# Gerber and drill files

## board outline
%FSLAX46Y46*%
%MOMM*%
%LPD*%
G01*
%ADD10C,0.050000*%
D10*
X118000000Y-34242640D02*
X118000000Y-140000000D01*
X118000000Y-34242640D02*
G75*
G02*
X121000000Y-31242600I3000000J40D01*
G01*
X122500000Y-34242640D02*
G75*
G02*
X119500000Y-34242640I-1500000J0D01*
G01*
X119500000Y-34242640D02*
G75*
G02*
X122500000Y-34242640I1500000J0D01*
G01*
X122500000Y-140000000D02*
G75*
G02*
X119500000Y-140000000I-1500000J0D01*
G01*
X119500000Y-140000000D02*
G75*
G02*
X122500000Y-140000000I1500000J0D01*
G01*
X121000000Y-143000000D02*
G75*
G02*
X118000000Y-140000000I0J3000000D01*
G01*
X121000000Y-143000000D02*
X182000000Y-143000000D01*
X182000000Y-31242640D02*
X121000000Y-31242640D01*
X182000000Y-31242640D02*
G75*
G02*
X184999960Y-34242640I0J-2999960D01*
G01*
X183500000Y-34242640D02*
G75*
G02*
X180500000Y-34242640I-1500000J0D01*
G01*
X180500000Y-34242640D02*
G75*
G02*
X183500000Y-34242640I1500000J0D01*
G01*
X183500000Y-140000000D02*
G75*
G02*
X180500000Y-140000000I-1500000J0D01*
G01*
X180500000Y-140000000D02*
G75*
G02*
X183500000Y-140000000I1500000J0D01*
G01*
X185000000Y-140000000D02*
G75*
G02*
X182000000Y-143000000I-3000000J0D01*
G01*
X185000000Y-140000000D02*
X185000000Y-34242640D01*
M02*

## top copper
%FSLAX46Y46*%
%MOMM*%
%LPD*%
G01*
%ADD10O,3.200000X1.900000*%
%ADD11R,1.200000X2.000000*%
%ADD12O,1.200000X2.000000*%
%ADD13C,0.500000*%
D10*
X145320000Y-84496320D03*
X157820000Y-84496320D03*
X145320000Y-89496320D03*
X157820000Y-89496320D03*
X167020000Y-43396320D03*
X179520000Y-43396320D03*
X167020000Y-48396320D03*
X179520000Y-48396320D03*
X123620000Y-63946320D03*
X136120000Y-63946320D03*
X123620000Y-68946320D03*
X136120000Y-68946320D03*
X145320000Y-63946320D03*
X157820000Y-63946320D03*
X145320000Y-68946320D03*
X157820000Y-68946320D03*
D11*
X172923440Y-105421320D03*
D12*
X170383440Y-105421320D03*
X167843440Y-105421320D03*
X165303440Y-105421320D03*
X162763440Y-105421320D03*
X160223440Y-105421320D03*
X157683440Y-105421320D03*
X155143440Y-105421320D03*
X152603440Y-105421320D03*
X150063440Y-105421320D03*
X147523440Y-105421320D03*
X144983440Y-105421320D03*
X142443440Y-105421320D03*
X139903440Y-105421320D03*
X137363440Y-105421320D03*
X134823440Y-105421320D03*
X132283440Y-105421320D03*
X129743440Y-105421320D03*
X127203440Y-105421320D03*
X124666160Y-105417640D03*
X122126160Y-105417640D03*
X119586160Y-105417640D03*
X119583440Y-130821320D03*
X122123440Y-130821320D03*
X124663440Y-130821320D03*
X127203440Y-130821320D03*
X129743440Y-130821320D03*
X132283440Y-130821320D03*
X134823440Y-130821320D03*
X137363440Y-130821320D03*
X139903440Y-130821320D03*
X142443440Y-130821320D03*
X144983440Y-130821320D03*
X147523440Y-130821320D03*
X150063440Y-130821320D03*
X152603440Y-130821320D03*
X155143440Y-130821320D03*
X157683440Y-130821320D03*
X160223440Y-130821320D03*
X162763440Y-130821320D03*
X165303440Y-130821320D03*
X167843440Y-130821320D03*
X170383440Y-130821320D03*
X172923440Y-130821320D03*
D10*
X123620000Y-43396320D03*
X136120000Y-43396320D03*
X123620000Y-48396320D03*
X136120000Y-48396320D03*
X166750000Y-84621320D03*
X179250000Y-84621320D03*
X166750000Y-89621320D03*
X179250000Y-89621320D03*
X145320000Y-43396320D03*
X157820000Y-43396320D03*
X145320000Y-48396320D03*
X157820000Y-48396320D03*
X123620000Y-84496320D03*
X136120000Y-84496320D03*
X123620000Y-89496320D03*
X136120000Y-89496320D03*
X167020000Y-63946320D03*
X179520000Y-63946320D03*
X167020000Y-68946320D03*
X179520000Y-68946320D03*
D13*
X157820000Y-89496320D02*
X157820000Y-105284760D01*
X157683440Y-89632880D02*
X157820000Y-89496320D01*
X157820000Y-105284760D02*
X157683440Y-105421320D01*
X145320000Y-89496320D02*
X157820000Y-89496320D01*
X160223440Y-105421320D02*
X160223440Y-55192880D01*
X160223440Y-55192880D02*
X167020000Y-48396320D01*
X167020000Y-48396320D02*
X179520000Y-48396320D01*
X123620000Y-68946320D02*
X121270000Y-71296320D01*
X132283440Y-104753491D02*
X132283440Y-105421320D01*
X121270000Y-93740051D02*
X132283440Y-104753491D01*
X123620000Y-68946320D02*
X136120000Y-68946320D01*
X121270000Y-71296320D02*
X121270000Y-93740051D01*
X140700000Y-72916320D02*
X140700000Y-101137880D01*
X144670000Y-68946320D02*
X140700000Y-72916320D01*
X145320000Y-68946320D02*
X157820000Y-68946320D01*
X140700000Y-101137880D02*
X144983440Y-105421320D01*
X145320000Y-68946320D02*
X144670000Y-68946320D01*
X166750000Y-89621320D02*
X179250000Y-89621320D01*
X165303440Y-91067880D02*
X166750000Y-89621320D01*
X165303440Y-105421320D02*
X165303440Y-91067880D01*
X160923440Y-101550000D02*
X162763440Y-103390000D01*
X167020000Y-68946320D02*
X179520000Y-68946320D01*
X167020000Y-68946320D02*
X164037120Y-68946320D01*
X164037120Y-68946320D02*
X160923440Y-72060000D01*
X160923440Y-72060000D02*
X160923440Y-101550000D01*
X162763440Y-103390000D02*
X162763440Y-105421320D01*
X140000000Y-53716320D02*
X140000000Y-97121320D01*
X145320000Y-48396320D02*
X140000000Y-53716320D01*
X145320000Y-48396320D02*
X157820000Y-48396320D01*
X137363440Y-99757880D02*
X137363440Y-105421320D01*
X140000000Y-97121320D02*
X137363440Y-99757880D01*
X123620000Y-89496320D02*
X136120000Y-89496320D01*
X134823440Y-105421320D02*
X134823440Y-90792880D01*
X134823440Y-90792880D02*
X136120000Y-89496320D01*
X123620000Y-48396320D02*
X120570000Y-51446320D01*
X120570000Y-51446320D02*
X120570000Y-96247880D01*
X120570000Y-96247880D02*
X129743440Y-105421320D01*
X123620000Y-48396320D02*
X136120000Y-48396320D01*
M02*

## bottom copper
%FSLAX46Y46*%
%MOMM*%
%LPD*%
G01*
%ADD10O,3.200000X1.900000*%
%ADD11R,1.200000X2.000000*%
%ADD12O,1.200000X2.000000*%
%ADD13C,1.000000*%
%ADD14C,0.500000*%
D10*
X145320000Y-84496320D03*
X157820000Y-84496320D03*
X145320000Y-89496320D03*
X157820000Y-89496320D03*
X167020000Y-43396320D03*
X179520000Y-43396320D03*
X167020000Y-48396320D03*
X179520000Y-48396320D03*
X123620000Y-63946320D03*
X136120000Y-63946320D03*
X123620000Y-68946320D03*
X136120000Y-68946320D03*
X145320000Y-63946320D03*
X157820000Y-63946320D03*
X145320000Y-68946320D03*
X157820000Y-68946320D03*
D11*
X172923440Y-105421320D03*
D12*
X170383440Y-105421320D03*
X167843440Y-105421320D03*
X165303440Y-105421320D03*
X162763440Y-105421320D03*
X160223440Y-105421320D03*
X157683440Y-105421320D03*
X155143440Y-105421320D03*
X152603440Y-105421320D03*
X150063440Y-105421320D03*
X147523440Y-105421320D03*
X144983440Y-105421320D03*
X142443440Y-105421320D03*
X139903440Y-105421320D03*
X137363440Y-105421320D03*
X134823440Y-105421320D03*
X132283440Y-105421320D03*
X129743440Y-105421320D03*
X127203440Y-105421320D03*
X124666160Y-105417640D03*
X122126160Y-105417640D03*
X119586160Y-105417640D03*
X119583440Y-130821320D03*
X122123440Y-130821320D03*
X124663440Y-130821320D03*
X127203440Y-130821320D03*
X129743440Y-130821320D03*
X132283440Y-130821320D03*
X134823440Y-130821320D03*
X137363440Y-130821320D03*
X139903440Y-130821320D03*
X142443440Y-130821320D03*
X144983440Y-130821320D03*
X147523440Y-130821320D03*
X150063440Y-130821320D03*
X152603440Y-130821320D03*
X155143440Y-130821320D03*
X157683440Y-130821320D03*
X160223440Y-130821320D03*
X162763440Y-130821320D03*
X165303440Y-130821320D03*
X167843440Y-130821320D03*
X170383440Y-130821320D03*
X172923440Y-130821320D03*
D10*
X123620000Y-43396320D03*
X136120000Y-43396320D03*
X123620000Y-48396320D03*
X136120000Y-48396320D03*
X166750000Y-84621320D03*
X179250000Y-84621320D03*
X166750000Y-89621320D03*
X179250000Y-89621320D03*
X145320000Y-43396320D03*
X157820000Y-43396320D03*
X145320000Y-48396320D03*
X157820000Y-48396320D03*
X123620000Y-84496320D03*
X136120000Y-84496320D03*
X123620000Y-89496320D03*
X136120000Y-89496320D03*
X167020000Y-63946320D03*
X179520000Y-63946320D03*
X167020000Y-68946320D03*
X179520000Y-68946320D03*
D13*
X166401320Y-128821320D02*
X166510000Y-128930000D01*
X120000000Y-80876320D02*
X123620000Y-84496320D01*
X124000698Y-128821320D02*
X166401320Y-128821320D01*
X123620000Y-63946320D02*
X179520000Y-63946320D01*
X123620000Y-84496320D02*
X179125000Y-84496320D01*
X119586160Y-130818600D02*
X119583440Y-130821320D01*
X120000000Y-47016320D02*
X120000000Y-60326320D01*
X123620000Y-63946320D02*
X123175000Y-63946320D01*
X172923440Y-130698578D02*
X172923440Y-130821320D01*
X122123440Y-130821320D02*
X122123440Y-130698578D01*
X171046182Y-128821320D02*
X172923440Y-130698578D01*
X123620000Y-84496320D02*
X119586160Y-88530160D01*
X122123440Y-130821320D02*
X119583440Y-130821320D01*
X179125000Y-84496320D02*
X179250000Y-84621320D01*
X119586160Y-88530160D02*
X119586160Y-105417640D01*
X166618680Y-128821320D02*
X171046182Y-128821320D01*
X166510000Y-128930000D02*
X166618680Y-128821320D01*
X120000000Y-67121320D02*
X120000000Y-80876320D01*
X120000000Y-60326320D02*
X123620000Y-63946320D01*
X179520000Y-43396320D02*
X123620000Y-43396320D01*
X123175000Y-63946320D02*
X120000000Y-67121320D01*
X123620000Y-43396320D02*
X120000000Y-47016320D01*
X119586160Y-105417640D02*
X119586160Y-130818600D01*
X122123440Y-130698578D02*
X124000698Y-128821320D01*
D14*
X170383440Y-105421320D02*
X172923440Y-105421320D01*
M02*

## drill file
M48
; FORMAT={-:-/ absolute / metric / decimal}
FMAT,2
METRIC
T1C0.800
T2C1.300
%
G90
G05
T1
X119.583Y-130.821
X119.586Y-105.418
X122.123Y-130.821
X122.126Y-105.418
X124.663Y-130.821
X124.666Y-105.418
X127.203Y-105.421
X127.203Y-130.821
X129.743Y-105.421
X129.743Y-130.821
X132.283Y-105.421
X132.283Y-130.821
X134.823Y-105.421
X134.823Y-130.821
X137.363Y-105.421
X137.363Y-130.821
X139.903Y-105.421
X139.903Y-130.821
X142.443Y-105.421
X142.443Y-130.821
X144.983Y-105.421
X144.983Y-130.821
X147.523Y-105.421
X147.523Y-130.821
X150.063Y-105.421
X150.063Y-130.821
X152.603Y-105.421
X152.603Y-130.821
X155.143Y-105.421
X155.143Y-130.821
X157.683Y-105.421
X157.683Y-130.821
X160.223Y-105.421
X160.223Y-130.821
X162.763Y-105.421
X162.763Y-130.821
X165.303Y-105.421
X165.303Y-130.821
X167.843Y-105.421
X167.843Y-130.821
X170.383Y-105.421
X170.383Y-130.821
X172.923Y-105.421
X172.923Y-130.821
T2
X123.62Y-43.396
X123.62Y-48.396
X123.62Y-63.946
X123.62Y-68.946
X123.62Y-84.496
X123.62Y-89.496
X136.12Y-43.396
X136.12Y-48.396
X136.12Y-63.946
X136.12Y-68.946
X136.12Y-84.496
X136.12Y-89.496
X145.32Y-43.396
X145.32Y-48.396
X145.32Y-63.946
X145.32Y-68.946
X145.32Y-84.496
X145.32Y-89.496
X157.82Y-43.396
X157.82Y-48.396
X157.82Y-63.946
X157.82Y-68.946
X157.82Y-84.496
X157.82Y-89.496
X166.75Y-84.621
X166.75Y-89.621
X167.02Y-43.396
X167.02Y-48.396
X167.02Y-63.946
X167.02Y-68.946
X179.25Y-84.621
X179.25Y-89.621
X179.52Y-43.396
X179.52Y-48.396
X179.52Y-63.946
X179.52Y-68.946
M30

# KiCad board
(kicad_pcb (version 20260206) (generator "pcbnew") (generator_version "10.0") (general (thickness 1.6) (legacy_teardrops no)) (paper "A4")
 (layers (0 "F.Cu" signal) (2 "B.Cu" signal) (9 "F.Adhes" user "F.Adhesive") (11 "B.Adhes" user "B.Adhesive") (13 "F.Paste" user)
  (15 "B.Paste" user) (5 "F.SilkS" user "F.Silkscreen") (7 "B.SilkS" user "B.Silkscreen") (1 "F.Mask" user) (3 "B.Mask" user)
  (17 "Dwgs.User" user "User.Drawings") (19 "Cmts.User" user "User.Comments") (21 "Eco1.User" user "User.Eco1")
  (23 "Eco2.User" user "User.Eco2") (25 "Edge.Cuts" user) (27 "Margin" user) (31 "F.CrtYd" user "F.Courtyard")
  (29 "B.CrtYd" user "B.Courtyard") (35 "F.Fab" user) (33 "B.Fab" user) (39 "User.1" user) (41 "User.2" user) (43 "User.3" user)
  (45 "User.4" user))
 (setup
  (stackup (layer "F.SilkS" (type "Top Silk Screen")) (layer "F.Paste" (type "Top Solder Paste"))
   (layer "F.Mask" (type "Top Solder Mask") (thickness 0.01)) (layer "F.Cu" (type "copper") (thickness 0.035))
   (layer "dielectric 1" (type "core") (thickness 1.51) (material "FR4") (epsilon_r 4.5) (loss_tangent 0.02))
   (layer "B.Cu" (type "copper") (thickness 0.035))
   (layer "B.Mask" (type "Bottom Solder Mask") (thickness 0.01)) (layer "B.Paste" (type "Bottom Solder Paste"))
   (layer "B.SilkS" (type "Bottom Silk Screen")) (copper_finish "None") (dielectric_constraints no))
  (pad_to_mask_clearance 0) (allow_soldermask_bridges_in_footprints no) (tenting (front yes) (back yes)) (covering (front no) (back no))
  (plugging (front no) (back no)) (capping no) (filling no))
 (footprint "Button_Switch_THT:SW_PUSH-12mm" (layer "F.Cu") (at 145.32 84.49632)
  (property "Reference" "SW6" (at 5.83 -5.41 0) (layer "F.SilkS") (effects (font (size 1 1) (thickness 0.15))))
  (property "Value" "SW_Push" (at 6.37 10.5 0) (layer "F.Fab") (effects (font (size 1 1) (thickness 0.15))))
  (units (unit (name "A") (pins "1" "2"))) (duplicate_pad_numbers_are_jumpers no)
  (pad "1" thru_hole oval (at 0 0) (size 3.2 1.9) (drill 1.3) (layers "*.Cu" "*.Mask") (remove_unused_layers no) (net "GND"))
  (pad "1" thru_hole oval (at 12.5 0) (size 3.2 1.9) (drill 1.3) (layers "*.Cu" "*.Mask") (remove_unused_layers no) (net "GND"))
  (pad "2" thru_hole oval (at 0 5) (size 3.2 1.9) (drill 1.3) (layers "*.Cu" "*.Mask") (remove_unused_layers no)
   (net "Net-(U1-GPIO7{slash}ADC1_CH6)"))
  (pad "2" thru_hole oval (at 12.5 5) (size 3.2 1.9) (drill 1.3) (layers "*.Cu" "*.Mask") (remove_unused_layers no)
   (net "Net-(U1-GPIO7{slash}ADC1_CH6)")))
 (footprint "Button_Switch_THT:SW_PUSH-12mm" (layer "F.Cu") (at 167.02 43.39632)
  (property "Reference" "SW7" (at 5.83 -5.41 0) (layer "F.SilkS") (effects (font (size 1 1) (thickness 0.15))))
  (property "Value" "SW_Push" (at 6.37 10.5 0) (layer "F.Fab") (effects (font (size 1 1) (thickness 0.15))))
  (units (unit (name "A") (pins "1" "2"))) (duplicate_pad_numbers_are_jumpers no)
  (pad "1" thru_hole oval (at 0 0) (size 3.2 1.9) (drill 1.3) (layers "*.Cu" "*.Mask") (remove_unused_layers no) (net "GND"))
  (pad "1" thru_hole oval (at 12.5 0) (size 3.2 1.9) (drill 1.3) (layers "*.Cu" "*.Mask") (remove_unused_layers no) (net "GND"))
  (pad "2" thru_hole oval (at 0 5) (size 3.2 1.9) (drill 1.3) (layers "*.Cu" "*.Mask") (remove_unused_layers no)
   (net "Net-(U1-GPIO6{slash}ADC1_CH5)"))
  (pad "2" thru_hole oval (at 12.5 5) (size 3.2 1.9) (drill 1.3) (layers "*.Cu" "*.Mask") (remove_unused_layers no)
   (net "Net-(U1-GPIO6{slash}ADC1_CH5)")))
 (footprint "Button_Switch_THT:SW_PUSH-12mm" (layer "F.Cu") (at 123.62 63.94632)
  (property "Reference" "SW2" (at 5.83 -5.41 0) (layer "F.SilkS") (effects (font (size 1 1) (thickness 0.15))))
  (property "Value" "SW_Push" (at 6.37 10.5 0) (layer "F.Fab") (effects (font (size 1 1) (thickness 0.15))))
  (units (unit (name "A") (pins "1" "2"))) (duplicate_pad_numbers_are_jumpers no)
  (pad "1" thru_hole oval (at 0 0) (size 3.2 1.9) (drill 1.3) (layers "*.Cu" "*.Mask") (remove_unused_layers no) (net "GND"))
  (pad "1" thru_hole oval (at 12.5 0) (size 3.2 1.9) (drill 1.3) (layers "*.Cu" "*.Mask") (remove_unused_layers no) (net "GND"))
  (pad "2" thru_hole oval (at 0 5) (size 3.2 1.9) (drill 1.3) (layers "*.Cu" "*.Mask") (remove_unused_layers no)
   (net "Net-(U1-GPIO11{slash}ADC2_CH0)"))
  (pad "2" thru_hole oval (at 12.5 5) (size 3.2 1.9) (drill 1.3) (layers "*.Cu" "*.Mask") (remove_unused_layers no)
   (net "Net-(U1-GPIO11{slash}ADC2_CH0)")))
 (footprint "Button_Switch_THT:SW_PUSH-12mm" (layer "F.Cu") (at 145.32 63.94632)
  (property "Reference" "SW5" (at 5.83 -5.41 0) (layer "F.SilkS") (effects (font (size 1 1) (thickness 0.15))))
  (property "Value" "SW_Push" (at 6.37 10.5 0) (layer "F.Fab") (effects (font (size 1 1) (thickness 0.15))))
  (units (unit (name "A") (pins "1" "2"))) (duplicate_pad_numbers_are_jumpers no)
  (pad "1" thru_hole oval (at 0 0) (size 3.2 1.9) (drill 1.3) (layers "*.Cu" "*.Mask") (remove_unused_layers no) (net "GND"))
  (pad "1" thru_hole oval (at 12.5 0) (size 3.2 1.9) (drill 1.3) (layers "*.Cu" "*.Mask") (remove_unused_layers no) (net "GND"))
  (pad "2" thru_hole oval (at 0 5) (size 3.2 1.9) (drill 1.3) (layers "*.Cu" "*.Mask") (remove_unused_layers no)
   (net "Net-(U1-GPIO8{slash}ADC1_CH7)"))
  (pad "2" thru_hole oval (at 12.5 5) (size 3.2 1.9) (drill 1.3) (layers "*.Cu" "*.Mask") (remove_unused_layers no)
   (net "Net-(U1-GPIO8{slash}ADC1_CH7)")))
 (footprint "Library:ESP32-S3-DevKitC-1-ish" (layer "F.Cu") (at 172.92344 105.42132 -90)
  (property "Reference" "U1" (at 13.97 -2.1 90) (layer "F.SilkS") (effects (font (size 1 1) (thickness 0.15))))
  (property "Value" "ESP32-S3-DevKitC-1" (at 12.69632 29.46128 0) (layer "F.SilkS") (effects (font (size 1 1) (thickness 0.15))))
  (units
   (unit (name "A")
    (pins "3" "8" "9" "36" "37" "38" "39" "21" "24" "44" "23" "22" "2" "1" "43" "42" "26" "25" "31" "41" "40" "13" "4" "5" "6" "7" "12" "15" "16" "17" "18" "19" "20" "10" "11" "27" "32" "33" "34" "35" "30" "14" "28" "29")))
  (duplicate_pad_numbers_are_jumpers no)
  (pad "1" thru_hole rect (at 0 0 180) (size 1.2 2) (drill 0.8) (layers "*.Cu" "*.Mask") (remove_unused_layers no) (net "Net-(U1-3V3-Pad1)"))
  (pad "2" thru_hole oval (at 0 2.54 180) (size 1.2 2) (drill 0.8) (layers "*.Cu" "*.Mask") (remove_unused_layers no)
   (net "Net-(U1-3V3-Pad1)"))
  (pad "3" thru_hole oval (at 0 5.08 180) (size 1.2 2) (drill 0.8) (layers "*.Cu" "*.Mask") (remove_unused_layers no)
   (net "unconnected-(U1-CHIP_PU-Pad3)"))
  (pad "4" thru_hole oval (at 0 7.62 180) (size 1.2 2) (drill 0.8) (layers "*.Cu" "*.Mask") (remove_unused_layers no)
   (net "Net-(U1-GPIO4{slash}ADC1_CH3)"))
  (pad "5" thru_hole oval (at 0 10.16 180) (size 1.2 2) (drill 0.8) (layers "*.Cu" "*.Mask") (remove_unused_layers no)
   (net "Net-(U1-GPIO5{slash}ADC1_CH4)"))
  (pad "6" thru_hole oval (at 0 12.7 180) (size 1.2 2) (drill 0.8) (layers "*.Cu" "*.Mask") (remove_unused_layers no)
   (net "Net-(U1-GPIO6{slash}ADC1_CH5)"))
  (pad "7" thru_hole oval (at 0 15.24 180) (size 1.2 2) (drill 0.8) (layers "*.Cu" "*.Mask") (remove_unused_layers no)
   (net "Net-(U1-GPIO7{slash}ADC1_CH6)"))
  (pad "8" thru_hole oval (at 0 17.78 180) (size 1.2 2) (drill 0.8) (layers "*.Cu" "*.Mask") (remove_unused_layers no)
   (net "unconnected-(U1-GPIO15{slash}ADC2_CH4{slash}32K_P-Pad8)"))
  (pad "9" thru_hole oval (at 0 20.32 180) (size 1.2 2) (drill 0.8) (layers "*.Cu" "*.Mask") (remove_unused_layers no)
   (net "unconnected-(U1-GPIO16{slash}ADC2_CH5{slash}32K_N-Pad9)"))
  (pad "10" thru_hole oval (at 0 22.86 180) (size 1.2 2) (drill 0.8) (layers "*.Cu" "*.Mask") (remove_unused_layers no)
   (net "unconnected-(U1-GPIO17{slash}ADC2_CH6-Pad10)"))
  (pad "11" thru_hole oval (at 0 25.4 180) (size 1.2 2) (drill 0.8) (layers "*.Cu" "*.Mask") (remove_unused_layers no)
   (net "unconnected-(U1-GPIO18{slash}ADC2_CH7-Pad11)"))
  (pad "12" thru_hole oval (at 0 27.94 180) (size 1.2 2) (drill 0.8) (layers "*.Cu" "*.Mask") (remove_unused_layers no)
   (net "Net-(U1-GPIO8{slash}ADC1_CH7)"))
  (pad "13" thru_hole oval (at 0 30.48 180) (size 1.2 2) (drill 0.8) (layers "*.Cu" "*.Mask") (remove_unused_layers no)
   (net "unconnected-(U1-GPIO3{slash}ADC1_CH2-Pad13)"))
  (pad "14" thru_hole oval (at 0 33.02 180) (size 1.2 2) (drill 0.8) (layers "*.Cu" "*.Mask") (remove_unused_layers no)
   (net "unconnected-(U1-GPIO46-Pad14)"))
  (pad "15" thru_hole oval (at 0 35.56 180) (size 1.2 2) (drill 0.8) (layers "*.Cu" "*.Mask") (remove_unused_layers no)
   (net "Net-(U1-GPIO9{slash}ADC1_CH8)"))
  (pad "16" thru_hole oval (at 0 38.1 180) (size 1.2 2) (drill 0.8) (layers "*.Cu" "*.Mask") (remove_unused_layers no)
   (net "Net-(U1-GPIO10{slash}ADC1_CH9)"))
  (pad "17" thru_hole oval (at 0 40.64 180) (size 1.2 2) (drill 0.8) (layers "*.Cu" "*.Mask") (remove_unused_layers no)
   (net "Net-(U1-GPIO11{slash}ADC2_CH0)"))
  (pad "18" thru_hole oval (at 0 43.18 180) (size 1.2 2) (drill 0.8) (layers "*.Cu" "*.Mask") (remove_unused_layers no)
   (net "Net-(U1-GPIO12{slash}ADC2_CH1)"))
  (pad "19" thru_hole oval (at 0 45.72 180) (size 1.2 2) (drill 0.8) (layers "*.Cu" "*.Mask") (remove_unused_layers no)
   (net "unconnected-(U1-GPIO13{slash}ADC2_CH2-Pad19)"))
  (pad "20" thru_hole oval (at -0.00368 48.25728 180) (size 1.2 2) (drill 0.8) (layers "*.Cu" "*.Mask") (remove_unused_layers no)
   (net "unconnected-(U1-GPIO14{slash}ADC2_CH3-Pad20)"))
  (pad "21" thru_hole oval (at -0.00368 50.79728 180) (size 1.2 2) (drill 0.8) (layers "*.Cu" "*.Mask") (remove_unused_layers no)
   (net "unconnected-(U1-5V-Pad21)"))
  (pad "22" thru_hole oval (at -0.00368 53.33728 180) (size 1.2 2) (drill 0.8) (layers "*.Cu" "*.Mask") (remove_unused_layers no)
   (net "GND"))
  (pad "23" thru_hole oval (at 25.4 53.34 180) (size 1.2 2) (drill 0.8) (layers "*.Cu" "*.Mask") (remove_unused_layers no) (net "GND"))
  (pad "24" thru_hole oval (at 25.4 50.8 180) (size 1.2 2) (drill 0.8) (layers "*.Cu" "*.Mask") (remove_unused_layers no) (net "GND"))
  (pad "25" thru_hole oval (at 25.4 48.26 180) (size 1.2 2) (drill 0.8) (layers "*.Cu" "*.Mask") (remove_unused_layers no)
   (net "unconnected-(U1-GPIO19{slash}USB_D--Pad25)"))
  (pad "26" thru_hole oval (at 25.4 45.72 180) (size 1.2 2) (drill 0.8) (layers "*.Cu" "*.Mask") (remove_unused_layers no)
   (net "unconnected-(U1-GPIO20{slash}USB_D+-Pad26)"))
  (pad "27" thru_hole oval (at 25.4 43.18 180) (size 1.2 2) (drill 0.8) (layers "*.Cu" "*.Mask") (remove_unused_layers no)
   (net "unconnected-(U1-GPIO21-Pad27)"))
  (pad "28" thru_hole oval (at 25.4 40.64 180) (size 1.2 2) (drill 0.8) (layers "*.Cu" "*.Mask") (remove_unused_layers no)
   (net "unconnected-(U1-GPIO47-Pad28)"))
  (pad "29" thru_hole oval (at 25.4 38.1 180) (size 1.2 2) (drill 0.8) (layers "*.Cu" "*.Mask") (remove_unused_layers no)
   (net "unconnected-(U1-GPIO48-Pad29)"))
  (pad "30" thru_hole oval (at 25.4 35.56 180) (size 1.2 2) (drill 0.8) (layers "*.Cu" "*.Mask") (remove_unused_layers no)
   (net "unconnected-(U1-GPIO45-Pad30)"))
  (pad "31" thru_hole oval (at 25.4 33.02 180) (size 1.2 2) (drill 0.8) (layers "*.Cu" "*.Mask") (remove_unused_layers no)
   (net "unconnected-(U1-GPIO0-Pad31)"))
  (pad "32" thru_hole oval (at 25.4 30.48 180) (size 1.2 2) (drill 0.8) (layers "*.Cu" "*.Mask") (remove_unused_layers no)
   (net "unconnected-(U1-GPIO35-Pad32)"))
  (pad "33" thru_hole oval (at 25.4 27.94 180) (size 1.2 2) (drill 0.8) (layers "*.Cu" "*.Mask") (remove_unused_layers no)
   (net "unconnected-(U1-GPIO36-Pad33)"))
  (pad "34" thru_hole oval (at 25.4 25.4 180) (size 1.2 2) (drill 0.8) (layers "*.Cu" "*.Mask") (remove_unused_layers no)
   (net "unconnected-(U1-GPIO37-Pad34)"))
  (pad "35" thru_hole oval (at 25.4 22.86 180) (size 1.2 2) (drill 0.8) (layers "*.Cu" "*.Mask") (remove_unused_layers no)
   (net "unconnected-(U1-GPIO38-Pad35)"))
  (pad "36" thru_hole oval (at 25.4 20.32 180) (size 1.2 2) (drill 0.8) (layers "*.Cu" "*.Mask") (remove_unused_layers no)
   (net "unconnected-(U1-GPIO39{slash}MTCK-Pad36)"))
  (pad "37" thru_hole oval (at 25.4 17.78 180) (size 1.2 2) (drill 0.8) (layers "*.Cu" "*.Mask") (remove_unused_layers no)
   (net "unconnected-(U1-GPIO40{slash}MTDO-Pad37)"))
  (pad "38" thru_hole oval (at 25.4 15.24 180) (size 1.2 2) (drill 0.8) (layers "*.Cu" "*.Mask") (remove_unused_layers no)
   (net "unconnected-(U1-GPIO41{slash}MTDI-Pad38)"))
  (pad "39" thru_hole oval (at 25.4 12.7 180) (size 1.2 2) (drill 0.8) (layers "*.Cu" "*.Mask") (remove_unused_layers no)
   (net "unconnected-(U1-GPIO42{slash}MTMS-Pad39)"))
  (pad "40" thru_hole oval (at 25.4 10.16 180) (size 1.2 2) (drill 0.8) (layers "*.Cu" "*.Mask") (remove_unused_layers no)
   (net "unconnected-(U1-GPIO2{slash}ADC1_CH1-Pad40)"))
  (pad "41" thru_hole oval (at 25.4 7.62 180) (size 1.2 2) (drill 0.8) (layers "*.Cu" "*.Mask") (remove_unused_layers no)
   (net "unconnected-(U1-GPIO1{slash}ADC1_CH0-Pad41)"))
  (pad "42" thru_hole oval (at 25.4 5.08 180) (size 1.2 2) (drill 0.8) (layers "*.Cu" "*.Mask") (remove_unused_layers no)
   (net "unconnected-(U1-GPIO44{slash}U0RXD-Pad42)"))
  (pad "43" thru_hole oval (at 25.4 2.54 180) (size 1.2 2) (drill 0.8) (layers "*.Cu" "*.Mask") (remove_unused_layers no)
   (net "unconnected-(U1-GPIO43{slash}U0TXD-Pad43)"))
  (pad "44" thru_hole oval (at 25.4 0 180) (size 1.2 2) (drill 0.8) (layers "*.Cu" "*.Mask") (remove_unused_layers no) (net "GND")))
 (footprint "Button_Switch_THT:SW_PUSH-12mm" (layer "F.Cu") (at 123.62 43.39632)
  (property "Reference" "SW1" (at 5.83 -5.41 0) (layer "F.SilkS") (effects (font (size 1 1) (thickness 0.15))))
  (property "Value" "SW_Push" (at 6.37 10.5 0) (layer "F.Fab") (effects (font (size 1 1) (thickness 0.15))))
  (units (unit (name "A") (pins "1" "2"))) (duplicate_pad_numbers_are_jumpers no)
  (pad "1" thru_hole oval (at 0 0) (size 3.2 1.9) (drill 1.3) (layers "*.Cu" "*.Mask") (remove_unused_layers no) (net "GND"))
  (pad "1" thru_hole oval (at 12.5 0) (size 3.2 1.9) (drill 1.3) (layers "*.Cu" "*.Mask") (remove_unused_layers no) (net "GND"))
  (pad "2" thru_hole oval (at 0 5) (size 3.2 1.9) (drill 1.3) (layers "*.Cu" "*.Mask") (remove_unused_layers no)
   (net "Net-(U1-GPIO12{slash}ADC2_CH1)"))
  (pad "2" thru_hole oval (at 12.5 5) (size 3.2 1.9) (drill 1.3) (layers "*.Cu" "*.Mask") (remove_unused_layers no)
   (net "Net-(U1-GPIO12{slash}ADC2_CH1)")))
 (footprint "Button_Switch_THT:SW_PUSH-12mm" (layer "F.Cu") (at 166.75 84.62132)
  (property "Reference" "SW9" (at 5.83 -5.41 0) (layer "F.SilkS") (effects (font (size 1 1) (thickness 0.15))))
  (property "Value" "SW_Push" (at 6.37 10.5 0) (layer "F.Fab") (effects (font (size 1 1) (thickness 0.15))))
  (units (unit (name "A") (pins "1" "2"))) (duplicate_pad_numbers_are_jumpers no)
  (pad "1" thru_hole oval (at 0 0) (size 3.2 1.9) (drill 1.3) (layers "*.Cu" "*.Mask") (remove_unused_layers no) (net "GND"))
  (pad "1" thru_hole oval (at 12.5 0) (size 3.2 1.9) (drill 1.3) (layers "*.Cu" "*.Mask") (remove_unused_layers no) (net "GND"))
  (pad "2" thru_hole oval (at 0 5) (size 3.2 1.9) (drill 1.3) (layers "*.Cu" "*.Mask") (remove_unused_layers no)
   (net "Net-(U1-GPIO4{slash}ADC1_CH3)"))
  (pad "2" thru_hole oval (at 12.5 5) (size 3.2 1.9) (drill 1.3) (layers "*.Cu" "*.Mask") (remove_unused_layers no)
   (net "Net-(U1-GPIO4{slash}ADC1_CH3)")))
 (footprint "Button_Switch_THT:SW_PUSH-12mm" (layer "F.Cu") (at 145.32 43.39632)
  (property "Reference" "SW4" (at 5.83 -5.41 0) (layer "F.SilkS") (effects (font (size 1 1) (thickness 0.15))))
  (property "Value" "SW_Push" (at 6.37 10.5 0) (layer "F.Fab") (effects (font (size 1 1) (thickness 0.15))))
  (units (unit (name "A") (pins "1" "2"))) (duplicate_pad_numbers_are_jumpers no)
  (pad "1" thru_hole oval (at 0 0) (size 3.2 1.9) (drill 1.3) (layers "*.Cu" "*.Mask") (remove_unused_layers no) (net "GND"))
  (pad "1" thru_hole oval (at 12.5 0) (size 3.2 1.9) (drill 1.3) (layers "*.Cu" "*.Mask") (remove_unused_layers no) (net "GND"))
  (pad "2" thru_hole oval (at 0 5) (size 3.2 1.9) (drill 1.3) (layers "*.Cu" "*.Mask") (remove_unused_layers no)
   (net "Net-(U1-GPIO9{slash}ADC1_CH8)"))
  (pad "2" thru_hole oval (at 12.5 5) (size 3.2 1.9) (drill 1.3) (layers "*.Cu" "*.Mask") (remove_unused_layers no)
   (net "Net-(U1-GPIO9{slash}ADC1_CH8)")))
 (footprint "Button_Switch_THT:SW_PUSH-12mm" (layer "F.Cu") (at 123.62 84.49632)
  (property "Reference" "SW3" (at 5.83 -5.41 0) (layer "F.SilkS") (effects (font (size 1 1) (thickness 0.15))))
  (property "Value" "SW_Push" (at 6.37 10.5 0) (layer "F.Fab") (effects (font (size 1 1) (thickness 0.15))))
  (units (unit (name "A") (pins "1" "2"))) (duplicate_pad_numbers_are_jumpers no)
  (pad "1" thru_hole oval (at 0 0) (size 3.2 1.9) (drill 1.3) (layers "*.Cu" "*.Mask") (remove_unused_layers no) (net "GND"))
  (pad "1" thru_hole oval (at 12.5 0) (size 3.2 1.9) (drill 1.3) (layers "*.Cu" "*.Mask") (remove_unused_layers no) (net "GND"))
  (pad "2" thru_hole oval (at 0 5) (size 3.2 1.9) (drill 1.3) (layers "*.Cu" "*.Mask") (remove_unused_layers no)
   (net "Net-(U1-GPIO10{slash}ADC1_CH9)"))
  (pad "2" thru_hole oval (at 12.5 5) (size 3.2 1.9) (drill 1.3) (layers "*.Cu" "*.Mask") (remove_unused_layers no)
   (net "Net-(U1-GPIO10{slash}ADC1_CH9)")))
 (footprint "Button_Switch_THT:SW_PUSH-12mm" (layer "F.Cu") (at 167.02 63.94632)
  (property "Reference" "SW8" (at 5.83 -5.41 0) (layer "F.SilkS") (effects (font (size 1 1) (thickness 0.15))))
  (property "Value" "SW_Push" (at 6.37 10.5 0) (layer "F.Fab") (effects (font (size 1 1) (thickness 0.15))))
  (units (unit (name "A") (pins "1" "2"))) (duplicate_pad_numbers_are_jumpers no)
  (pad "1" thru_hole oval (at 0 0) (size 3.2 1.9) (drill 1.3) (layers "*.Cu" "*.Mask") (remove_unused_layers no) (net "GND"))
  (pad "1" thru_hole oval (at 12.5 0) (size 3.2 1.9) (drill 1.3) (layers "*.Cu" "*.Mask") (remove_unused_layers no) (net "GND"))
  (pad "2" thru_hole oval (at 0 5) (size 3.2 1.9) (drill 1.3) (layers "*.Cu" "*.Mask") (remove_unused_layers no)
   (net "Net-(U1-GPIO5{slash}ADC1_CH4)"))
  (pad "2" thru_hole oval (at 12.5 5) (size 3.2 1.9) (drill 1.3) (layers "*.Cu" "*.Mask") (remove_unused_layers no)
   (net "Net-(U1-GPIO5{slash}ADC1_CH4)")))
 (gr_line (start 118 34.24264) (end 118 140) (stroke (width 0.05) (type default)) (layer "Edge.Cuts"))
 (gr_arc (start 118 34.24264) (mid 118.87868 32.12132) (end 121 31.24264) (stroke (width 0.05) (type default)) (layer "Edge.Cuts"))
 (gr_circle (center 121 34.24264) (end 122.5 34.24264) (stroke (width 0.05) (type solid)) (fill no) (layer "Edge.Cuts"))
 (gr_circle (center 121 140) (end 122.5 140) (stroke (width 0.05) (type solid)) (fill no) (layer "Edge.Cuts"))
 (gr_arc (start 121 143) (mid 118.87868 142.12132) (end 118 140) (stroke (width 0.05) (type default)) (layer "Edge.Cuts"))
 (gr_line (start 121 143) (end 182 143) (stroke (width 0.05) (type default)) (layer "Edge.Cuts"))
 (gr_line (start 182 31.24264) (end 121 31.24264) (stroke (width 0.05) (type default)) (layer "Edge.Cuts"))
 (gr_arc (start 182 31.24264) (mid 184.12132 32.12132) (end 185 34.24264) (stroke (width 0.05) (type default)) (layer "Edge.Cuts"))
 (gr_circle (center 182 34.24264) (end 183.5 34.24264) (stroke (width 0.05) (type solid)) (fill no) (layer "Edge.Cuts"))
 (gr_circle (center 182 140) (end 183.5 140) (stroke (width 0.05) (type solid)) (fill no) (layer "Edge.Cuts"))
 (gr_arc (start 185 140) (mid 184.12132 142.12132) (end 182 143) (stroke (width 0.05) (type default)) (layer "Edge.Cuts"))
 (gr_line (start 185 140) (end 185 34.24264) (stroke (width 0.05) (type default)) (layer "Edge.Cuts"))
 (segment (start 166.40132 128.82132) (end 166.51 128.93) (width 1) (layer "B.Cu") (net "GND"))
 (segment (start 120 80.87632) (end 123.62 84.49632) (width 1) (layer "B.Cu") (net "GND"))
 (segment (start 124.000698 128.82132) (end 166.40132 128.82132) (width 1) (layer "B.Cu") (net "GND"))
 (segment (start 123.62 63.94632) (end 179.52 63.94632) (width 1) (layer "B.Cu") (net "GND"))
 (segment (start 123.62 84.49632) (end 179.125 84.49632) (width 1) (layer "B.Cu") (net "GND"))
 (segment (start 119.58616 130.8186) (end 119.58344 130.82132) (width 1) (layer "B.Cu") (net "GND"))
 (segment (start 120 47.01632) (end 120 60.32632) (width 1) (layer "B.Cu") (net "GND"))
 (segment (start 123.62 63.94632) (end 123.175 63.94632) (width 1) (layer "B.Cu") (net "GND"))
 (segment (start 172.92344 130.698578) (end 172.92344 130.82132) (width 1) (layer "B.Cu") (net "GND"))
 (segment (start 122.12344 130.82132) (end 122.12344 130.698578) (width 1) (layer "B.Cu") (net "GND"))
 (segment (start 171.046182 128.82132) (end 172.92344 130.698578) (width 1) (layer "B.Cu") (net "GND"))
 (segment (start 123.62 84.49632) (end 119.58616 88.53016) (width 1) (layer "B.Cu") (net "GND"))
 (segment (start 122.12344 130.82132) (end 119.58344 130.82132) (width 1) (layer "B.Cu") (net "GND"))
 (segment (start 179.125 84.49632) (end 179.25 84.62132) (width 1) (layer "B.Cu") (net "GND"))
 (segment (start 119.58616 88.53016) (end 119.58616 105.41764) (width 1) (layer "B.Cu") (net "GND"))
 (segment (start 166.61868 128.82132) (end 171.046182 128.82132) (width 1) (layer "B.Cu") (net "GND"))
 (segment (start 166.51 128.93) (end 166.61868 128.82132) (width 1) (layer "B.Cu") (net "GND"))
 (segment (start 120 67.12132) (end 120 80.87632) (width 1) (layer "B.Cu") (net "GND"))
 (segment (start 120 60.32632) (end 123.62 63.94632) (width 1) (layer "B.Cu") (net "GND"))
 (segment (start 179.52 43.39632) (end 123.62 43.39632) (width 1) (layer "B.Cu") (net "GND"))
 (segment (start 123.175 63.94632) (end 120 67.12132) (width 1) (layer "B.Cu") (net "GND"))
 (segment (start 123.62 43.39632) (end 120 47.01632) (width 1) (layer "B.Cu") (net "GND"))
 (segment (start 119.58616 105.41764) (end 119.58616 130.8186) (width 1) (layer "B.Cu") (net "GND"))
 (segment (start 122.12344 130.698578) (end 124.000698 128.82132) (width 1) (layer "B.Cu") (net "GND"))
 (segment (start 157.82 89.49632) (end 157.82 105.28476) (width 0.5) (layer "F.Cu") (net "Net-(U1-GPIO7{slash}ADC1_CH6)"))
 (segment (start 157.68344 89.63288) (end 157.82 89.49632) (width 0.5) (layer "F.Cu") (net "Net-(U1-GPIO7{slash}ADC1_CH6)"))
 (segment (start 157.82 105.28476) (end 157.68344 105.42132) (width 0.5) (layer "F.Cu") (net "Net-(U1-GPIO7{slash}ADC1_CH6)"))
 (segment (start 145.32 89.49632) (end 157.82 89.49632) (width 0.5) (layer "F.Cu") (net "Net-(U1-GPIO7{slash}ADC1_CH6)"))
 (segment (start 160.22344 105.42132) (end 160.22344 55.19288) (width 0.5) (layer "F.Cu") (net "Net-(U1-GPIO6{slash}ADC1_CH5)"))
 (segment (start 160.22344 55.19288) (end 167.02 48.39632) (width 0.5) (layer "F.Cu") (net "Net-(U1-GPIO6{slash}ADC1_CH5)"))
 (segment (start 167.02 48.39632) (end 179.52 48.39632) (width 0.5) (layer "F.Cu") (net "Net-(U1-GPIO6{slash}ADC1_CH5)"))
 (segment (start 123.62 68.94632) (end 121.27 71.29632) (width 0.5) (layer "F.Cu") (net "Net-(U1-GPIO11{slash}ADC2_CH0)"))
 (segment (start 132.28344 104.753491) (end 132.28344 105.42132) (width 0.5) (layer "F.Cu") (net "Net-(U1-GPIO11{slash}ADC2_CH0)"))
 (segment (start 121.27 93.740051) (end 132.28344 104.753491) (width 0.5) (layer "F.Cu") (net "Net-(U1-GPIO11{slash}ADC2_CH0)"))
 (segment (start 123.62 68.94632) (end 136.12 68.94632) (width 0.5) (layer "F.Cu") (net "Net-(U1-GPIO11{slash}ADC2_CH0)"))
 (segment (start 121.27 71.29632) (end 121.27 93.740051) (width 0.5) (layer "F.Cu") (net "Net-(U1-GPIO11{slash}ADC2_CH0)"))
 (segment (start 140.7 72.91632) (end 140.7 101.13788) (width 0.5) (layer "F.Cu") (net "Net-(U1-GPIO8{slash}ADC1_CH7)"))
 (segment (start 144.67 68.94632) (end 140.7 72.91632) (width 0.5) (layer "F.Cu") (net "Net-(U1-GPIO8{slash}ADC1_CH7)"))
 (segment (start 145.32 68.94632) (end 157.82 68.94632) (width 0.5) (layer "F.Cu") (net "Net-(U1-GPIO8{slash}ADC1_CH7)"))
 (segment (start 140.7 101.13788) (end 144.98344 105.42132) (width 0.5) (layer "F.Cu") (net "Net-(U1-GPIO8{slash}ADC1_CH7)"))
 (segment (start 145.32 68.94632) (end 144.67 68.94632) (width 0.5) (layer "F.Cu") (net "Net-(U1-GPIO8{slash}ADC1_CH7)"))
 (segment (start 170.38344 105.42132) (end 172.92344 105.42132) (width 0.5) (layer "B.Cu") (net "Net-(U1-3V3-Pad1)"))
 (segment (start 166.75 89.62132) (end 179.25 89.62132) (width 0.5) (layer "F.Cu") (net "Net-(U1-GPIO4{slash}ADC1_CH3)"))
 (segment (start 165.30344 91.06788) (end 166.75 89.62132) (width 0.5) (layer "F.Cu") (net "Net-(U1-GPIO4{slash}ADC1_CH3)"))
 (segment (start 165.30344 105.42132) (end 165.30344 91.06788) (width 0.5) (layer "F.Cu") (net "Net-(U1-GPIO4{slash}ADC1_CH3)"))
 (segment (start 160.92344 101.55) (end 162.76344 103.39) (width 0.5) (layer "F.Cu") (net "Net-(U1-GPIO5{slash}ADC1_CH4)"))
 (segment (start 167.02 68.94632) (end 179.52 68.94632) (width 0.5) (layer "F.Cu") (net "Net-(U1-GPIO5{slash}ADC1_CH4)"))
 (segment (start 167.02 68.94632) (end 164.03712 68.94632) (width 0.5) (layer "F.Cu") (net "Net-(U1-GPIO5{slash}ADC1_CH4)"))
 (segment (start 164.03712 68.94632) (end 160.92344 72.06) (width 0.5) (layer "F.Cu") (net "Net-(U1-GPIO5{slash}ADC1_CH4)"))
 (segment (start 160.92344 72.06) (end 160.92344 101.55) (width 0.5) (layer "F.Cu") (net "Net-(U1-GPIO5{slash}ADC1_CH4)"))
 (segment (start 162.76344 103.39) (end 162.76344 105.42132) (width 0.5) (layer "F.Cu") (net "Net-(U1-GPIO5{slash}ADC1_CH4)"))
 (segment (start 140 53.71632) (end 140 97.12132) (width 0.5) (layer "F.Cu") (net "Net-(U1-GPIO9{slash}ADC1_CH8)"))
 (segment (start 145.32 48.39632) (end 140 53.71632) (width 0.5) (layer "F.Cu") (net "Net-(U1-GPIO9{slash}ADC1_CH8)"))
 (segment (start 145.32 48.39632) (end 157.82 48.39632) (width 0.5) (layer "F.Cu") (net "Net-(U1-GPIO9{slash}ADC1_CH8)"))
 (segment (start 137.36344 99.75788) (end 137.36344 105.42132) (width 0.5) (layer "F.Cu") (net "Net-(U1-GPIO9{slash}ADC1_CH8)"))
 (segment (start 140 97.12132) (end 137.36344 99.75788) (width 0.5) (layer "F.Cu") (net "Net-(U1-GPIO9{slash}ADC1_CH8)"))
 (segment (start 123.62 89.49632) (end 136.12 89.49632) (width 0.5) (layer "F.Cu") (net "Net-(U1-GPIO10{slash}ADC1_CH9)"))
 (segment (start 134.82344 105.42132) (end 134.82344 90.79288) (width 0.5) (layer "F.Cu") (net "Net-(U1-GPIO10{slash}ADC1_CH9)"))
 (segment (start 134.82344 90.79288) (end 136.12 89.49632) (width 0.5) (layer "F.Cu") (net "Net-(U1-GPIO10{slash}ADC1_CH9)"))
 (segment (start 123.62 48.39632) (end 120.57 51.44632) (width 0.5) (layer "F.Cu") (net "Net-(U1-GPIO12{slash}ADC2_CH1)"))
 (segment (start 120.57 51.44632) (end 120.57 96.24788) (width 0.5) (layer "F.Cu") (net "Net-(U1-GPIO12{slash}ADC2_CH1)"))
 (segment (start 120.57 96.24788) (end 129.74344 105.42132) (width 0.5) (layer "F.Cu") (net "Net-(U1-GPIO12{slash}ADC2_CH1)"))
 (segment (start 123.62 48.39632) (end 136.12 48.39632) (width 0.5) (layer "F.Cu") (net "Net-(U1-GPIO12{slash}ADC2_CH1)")))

